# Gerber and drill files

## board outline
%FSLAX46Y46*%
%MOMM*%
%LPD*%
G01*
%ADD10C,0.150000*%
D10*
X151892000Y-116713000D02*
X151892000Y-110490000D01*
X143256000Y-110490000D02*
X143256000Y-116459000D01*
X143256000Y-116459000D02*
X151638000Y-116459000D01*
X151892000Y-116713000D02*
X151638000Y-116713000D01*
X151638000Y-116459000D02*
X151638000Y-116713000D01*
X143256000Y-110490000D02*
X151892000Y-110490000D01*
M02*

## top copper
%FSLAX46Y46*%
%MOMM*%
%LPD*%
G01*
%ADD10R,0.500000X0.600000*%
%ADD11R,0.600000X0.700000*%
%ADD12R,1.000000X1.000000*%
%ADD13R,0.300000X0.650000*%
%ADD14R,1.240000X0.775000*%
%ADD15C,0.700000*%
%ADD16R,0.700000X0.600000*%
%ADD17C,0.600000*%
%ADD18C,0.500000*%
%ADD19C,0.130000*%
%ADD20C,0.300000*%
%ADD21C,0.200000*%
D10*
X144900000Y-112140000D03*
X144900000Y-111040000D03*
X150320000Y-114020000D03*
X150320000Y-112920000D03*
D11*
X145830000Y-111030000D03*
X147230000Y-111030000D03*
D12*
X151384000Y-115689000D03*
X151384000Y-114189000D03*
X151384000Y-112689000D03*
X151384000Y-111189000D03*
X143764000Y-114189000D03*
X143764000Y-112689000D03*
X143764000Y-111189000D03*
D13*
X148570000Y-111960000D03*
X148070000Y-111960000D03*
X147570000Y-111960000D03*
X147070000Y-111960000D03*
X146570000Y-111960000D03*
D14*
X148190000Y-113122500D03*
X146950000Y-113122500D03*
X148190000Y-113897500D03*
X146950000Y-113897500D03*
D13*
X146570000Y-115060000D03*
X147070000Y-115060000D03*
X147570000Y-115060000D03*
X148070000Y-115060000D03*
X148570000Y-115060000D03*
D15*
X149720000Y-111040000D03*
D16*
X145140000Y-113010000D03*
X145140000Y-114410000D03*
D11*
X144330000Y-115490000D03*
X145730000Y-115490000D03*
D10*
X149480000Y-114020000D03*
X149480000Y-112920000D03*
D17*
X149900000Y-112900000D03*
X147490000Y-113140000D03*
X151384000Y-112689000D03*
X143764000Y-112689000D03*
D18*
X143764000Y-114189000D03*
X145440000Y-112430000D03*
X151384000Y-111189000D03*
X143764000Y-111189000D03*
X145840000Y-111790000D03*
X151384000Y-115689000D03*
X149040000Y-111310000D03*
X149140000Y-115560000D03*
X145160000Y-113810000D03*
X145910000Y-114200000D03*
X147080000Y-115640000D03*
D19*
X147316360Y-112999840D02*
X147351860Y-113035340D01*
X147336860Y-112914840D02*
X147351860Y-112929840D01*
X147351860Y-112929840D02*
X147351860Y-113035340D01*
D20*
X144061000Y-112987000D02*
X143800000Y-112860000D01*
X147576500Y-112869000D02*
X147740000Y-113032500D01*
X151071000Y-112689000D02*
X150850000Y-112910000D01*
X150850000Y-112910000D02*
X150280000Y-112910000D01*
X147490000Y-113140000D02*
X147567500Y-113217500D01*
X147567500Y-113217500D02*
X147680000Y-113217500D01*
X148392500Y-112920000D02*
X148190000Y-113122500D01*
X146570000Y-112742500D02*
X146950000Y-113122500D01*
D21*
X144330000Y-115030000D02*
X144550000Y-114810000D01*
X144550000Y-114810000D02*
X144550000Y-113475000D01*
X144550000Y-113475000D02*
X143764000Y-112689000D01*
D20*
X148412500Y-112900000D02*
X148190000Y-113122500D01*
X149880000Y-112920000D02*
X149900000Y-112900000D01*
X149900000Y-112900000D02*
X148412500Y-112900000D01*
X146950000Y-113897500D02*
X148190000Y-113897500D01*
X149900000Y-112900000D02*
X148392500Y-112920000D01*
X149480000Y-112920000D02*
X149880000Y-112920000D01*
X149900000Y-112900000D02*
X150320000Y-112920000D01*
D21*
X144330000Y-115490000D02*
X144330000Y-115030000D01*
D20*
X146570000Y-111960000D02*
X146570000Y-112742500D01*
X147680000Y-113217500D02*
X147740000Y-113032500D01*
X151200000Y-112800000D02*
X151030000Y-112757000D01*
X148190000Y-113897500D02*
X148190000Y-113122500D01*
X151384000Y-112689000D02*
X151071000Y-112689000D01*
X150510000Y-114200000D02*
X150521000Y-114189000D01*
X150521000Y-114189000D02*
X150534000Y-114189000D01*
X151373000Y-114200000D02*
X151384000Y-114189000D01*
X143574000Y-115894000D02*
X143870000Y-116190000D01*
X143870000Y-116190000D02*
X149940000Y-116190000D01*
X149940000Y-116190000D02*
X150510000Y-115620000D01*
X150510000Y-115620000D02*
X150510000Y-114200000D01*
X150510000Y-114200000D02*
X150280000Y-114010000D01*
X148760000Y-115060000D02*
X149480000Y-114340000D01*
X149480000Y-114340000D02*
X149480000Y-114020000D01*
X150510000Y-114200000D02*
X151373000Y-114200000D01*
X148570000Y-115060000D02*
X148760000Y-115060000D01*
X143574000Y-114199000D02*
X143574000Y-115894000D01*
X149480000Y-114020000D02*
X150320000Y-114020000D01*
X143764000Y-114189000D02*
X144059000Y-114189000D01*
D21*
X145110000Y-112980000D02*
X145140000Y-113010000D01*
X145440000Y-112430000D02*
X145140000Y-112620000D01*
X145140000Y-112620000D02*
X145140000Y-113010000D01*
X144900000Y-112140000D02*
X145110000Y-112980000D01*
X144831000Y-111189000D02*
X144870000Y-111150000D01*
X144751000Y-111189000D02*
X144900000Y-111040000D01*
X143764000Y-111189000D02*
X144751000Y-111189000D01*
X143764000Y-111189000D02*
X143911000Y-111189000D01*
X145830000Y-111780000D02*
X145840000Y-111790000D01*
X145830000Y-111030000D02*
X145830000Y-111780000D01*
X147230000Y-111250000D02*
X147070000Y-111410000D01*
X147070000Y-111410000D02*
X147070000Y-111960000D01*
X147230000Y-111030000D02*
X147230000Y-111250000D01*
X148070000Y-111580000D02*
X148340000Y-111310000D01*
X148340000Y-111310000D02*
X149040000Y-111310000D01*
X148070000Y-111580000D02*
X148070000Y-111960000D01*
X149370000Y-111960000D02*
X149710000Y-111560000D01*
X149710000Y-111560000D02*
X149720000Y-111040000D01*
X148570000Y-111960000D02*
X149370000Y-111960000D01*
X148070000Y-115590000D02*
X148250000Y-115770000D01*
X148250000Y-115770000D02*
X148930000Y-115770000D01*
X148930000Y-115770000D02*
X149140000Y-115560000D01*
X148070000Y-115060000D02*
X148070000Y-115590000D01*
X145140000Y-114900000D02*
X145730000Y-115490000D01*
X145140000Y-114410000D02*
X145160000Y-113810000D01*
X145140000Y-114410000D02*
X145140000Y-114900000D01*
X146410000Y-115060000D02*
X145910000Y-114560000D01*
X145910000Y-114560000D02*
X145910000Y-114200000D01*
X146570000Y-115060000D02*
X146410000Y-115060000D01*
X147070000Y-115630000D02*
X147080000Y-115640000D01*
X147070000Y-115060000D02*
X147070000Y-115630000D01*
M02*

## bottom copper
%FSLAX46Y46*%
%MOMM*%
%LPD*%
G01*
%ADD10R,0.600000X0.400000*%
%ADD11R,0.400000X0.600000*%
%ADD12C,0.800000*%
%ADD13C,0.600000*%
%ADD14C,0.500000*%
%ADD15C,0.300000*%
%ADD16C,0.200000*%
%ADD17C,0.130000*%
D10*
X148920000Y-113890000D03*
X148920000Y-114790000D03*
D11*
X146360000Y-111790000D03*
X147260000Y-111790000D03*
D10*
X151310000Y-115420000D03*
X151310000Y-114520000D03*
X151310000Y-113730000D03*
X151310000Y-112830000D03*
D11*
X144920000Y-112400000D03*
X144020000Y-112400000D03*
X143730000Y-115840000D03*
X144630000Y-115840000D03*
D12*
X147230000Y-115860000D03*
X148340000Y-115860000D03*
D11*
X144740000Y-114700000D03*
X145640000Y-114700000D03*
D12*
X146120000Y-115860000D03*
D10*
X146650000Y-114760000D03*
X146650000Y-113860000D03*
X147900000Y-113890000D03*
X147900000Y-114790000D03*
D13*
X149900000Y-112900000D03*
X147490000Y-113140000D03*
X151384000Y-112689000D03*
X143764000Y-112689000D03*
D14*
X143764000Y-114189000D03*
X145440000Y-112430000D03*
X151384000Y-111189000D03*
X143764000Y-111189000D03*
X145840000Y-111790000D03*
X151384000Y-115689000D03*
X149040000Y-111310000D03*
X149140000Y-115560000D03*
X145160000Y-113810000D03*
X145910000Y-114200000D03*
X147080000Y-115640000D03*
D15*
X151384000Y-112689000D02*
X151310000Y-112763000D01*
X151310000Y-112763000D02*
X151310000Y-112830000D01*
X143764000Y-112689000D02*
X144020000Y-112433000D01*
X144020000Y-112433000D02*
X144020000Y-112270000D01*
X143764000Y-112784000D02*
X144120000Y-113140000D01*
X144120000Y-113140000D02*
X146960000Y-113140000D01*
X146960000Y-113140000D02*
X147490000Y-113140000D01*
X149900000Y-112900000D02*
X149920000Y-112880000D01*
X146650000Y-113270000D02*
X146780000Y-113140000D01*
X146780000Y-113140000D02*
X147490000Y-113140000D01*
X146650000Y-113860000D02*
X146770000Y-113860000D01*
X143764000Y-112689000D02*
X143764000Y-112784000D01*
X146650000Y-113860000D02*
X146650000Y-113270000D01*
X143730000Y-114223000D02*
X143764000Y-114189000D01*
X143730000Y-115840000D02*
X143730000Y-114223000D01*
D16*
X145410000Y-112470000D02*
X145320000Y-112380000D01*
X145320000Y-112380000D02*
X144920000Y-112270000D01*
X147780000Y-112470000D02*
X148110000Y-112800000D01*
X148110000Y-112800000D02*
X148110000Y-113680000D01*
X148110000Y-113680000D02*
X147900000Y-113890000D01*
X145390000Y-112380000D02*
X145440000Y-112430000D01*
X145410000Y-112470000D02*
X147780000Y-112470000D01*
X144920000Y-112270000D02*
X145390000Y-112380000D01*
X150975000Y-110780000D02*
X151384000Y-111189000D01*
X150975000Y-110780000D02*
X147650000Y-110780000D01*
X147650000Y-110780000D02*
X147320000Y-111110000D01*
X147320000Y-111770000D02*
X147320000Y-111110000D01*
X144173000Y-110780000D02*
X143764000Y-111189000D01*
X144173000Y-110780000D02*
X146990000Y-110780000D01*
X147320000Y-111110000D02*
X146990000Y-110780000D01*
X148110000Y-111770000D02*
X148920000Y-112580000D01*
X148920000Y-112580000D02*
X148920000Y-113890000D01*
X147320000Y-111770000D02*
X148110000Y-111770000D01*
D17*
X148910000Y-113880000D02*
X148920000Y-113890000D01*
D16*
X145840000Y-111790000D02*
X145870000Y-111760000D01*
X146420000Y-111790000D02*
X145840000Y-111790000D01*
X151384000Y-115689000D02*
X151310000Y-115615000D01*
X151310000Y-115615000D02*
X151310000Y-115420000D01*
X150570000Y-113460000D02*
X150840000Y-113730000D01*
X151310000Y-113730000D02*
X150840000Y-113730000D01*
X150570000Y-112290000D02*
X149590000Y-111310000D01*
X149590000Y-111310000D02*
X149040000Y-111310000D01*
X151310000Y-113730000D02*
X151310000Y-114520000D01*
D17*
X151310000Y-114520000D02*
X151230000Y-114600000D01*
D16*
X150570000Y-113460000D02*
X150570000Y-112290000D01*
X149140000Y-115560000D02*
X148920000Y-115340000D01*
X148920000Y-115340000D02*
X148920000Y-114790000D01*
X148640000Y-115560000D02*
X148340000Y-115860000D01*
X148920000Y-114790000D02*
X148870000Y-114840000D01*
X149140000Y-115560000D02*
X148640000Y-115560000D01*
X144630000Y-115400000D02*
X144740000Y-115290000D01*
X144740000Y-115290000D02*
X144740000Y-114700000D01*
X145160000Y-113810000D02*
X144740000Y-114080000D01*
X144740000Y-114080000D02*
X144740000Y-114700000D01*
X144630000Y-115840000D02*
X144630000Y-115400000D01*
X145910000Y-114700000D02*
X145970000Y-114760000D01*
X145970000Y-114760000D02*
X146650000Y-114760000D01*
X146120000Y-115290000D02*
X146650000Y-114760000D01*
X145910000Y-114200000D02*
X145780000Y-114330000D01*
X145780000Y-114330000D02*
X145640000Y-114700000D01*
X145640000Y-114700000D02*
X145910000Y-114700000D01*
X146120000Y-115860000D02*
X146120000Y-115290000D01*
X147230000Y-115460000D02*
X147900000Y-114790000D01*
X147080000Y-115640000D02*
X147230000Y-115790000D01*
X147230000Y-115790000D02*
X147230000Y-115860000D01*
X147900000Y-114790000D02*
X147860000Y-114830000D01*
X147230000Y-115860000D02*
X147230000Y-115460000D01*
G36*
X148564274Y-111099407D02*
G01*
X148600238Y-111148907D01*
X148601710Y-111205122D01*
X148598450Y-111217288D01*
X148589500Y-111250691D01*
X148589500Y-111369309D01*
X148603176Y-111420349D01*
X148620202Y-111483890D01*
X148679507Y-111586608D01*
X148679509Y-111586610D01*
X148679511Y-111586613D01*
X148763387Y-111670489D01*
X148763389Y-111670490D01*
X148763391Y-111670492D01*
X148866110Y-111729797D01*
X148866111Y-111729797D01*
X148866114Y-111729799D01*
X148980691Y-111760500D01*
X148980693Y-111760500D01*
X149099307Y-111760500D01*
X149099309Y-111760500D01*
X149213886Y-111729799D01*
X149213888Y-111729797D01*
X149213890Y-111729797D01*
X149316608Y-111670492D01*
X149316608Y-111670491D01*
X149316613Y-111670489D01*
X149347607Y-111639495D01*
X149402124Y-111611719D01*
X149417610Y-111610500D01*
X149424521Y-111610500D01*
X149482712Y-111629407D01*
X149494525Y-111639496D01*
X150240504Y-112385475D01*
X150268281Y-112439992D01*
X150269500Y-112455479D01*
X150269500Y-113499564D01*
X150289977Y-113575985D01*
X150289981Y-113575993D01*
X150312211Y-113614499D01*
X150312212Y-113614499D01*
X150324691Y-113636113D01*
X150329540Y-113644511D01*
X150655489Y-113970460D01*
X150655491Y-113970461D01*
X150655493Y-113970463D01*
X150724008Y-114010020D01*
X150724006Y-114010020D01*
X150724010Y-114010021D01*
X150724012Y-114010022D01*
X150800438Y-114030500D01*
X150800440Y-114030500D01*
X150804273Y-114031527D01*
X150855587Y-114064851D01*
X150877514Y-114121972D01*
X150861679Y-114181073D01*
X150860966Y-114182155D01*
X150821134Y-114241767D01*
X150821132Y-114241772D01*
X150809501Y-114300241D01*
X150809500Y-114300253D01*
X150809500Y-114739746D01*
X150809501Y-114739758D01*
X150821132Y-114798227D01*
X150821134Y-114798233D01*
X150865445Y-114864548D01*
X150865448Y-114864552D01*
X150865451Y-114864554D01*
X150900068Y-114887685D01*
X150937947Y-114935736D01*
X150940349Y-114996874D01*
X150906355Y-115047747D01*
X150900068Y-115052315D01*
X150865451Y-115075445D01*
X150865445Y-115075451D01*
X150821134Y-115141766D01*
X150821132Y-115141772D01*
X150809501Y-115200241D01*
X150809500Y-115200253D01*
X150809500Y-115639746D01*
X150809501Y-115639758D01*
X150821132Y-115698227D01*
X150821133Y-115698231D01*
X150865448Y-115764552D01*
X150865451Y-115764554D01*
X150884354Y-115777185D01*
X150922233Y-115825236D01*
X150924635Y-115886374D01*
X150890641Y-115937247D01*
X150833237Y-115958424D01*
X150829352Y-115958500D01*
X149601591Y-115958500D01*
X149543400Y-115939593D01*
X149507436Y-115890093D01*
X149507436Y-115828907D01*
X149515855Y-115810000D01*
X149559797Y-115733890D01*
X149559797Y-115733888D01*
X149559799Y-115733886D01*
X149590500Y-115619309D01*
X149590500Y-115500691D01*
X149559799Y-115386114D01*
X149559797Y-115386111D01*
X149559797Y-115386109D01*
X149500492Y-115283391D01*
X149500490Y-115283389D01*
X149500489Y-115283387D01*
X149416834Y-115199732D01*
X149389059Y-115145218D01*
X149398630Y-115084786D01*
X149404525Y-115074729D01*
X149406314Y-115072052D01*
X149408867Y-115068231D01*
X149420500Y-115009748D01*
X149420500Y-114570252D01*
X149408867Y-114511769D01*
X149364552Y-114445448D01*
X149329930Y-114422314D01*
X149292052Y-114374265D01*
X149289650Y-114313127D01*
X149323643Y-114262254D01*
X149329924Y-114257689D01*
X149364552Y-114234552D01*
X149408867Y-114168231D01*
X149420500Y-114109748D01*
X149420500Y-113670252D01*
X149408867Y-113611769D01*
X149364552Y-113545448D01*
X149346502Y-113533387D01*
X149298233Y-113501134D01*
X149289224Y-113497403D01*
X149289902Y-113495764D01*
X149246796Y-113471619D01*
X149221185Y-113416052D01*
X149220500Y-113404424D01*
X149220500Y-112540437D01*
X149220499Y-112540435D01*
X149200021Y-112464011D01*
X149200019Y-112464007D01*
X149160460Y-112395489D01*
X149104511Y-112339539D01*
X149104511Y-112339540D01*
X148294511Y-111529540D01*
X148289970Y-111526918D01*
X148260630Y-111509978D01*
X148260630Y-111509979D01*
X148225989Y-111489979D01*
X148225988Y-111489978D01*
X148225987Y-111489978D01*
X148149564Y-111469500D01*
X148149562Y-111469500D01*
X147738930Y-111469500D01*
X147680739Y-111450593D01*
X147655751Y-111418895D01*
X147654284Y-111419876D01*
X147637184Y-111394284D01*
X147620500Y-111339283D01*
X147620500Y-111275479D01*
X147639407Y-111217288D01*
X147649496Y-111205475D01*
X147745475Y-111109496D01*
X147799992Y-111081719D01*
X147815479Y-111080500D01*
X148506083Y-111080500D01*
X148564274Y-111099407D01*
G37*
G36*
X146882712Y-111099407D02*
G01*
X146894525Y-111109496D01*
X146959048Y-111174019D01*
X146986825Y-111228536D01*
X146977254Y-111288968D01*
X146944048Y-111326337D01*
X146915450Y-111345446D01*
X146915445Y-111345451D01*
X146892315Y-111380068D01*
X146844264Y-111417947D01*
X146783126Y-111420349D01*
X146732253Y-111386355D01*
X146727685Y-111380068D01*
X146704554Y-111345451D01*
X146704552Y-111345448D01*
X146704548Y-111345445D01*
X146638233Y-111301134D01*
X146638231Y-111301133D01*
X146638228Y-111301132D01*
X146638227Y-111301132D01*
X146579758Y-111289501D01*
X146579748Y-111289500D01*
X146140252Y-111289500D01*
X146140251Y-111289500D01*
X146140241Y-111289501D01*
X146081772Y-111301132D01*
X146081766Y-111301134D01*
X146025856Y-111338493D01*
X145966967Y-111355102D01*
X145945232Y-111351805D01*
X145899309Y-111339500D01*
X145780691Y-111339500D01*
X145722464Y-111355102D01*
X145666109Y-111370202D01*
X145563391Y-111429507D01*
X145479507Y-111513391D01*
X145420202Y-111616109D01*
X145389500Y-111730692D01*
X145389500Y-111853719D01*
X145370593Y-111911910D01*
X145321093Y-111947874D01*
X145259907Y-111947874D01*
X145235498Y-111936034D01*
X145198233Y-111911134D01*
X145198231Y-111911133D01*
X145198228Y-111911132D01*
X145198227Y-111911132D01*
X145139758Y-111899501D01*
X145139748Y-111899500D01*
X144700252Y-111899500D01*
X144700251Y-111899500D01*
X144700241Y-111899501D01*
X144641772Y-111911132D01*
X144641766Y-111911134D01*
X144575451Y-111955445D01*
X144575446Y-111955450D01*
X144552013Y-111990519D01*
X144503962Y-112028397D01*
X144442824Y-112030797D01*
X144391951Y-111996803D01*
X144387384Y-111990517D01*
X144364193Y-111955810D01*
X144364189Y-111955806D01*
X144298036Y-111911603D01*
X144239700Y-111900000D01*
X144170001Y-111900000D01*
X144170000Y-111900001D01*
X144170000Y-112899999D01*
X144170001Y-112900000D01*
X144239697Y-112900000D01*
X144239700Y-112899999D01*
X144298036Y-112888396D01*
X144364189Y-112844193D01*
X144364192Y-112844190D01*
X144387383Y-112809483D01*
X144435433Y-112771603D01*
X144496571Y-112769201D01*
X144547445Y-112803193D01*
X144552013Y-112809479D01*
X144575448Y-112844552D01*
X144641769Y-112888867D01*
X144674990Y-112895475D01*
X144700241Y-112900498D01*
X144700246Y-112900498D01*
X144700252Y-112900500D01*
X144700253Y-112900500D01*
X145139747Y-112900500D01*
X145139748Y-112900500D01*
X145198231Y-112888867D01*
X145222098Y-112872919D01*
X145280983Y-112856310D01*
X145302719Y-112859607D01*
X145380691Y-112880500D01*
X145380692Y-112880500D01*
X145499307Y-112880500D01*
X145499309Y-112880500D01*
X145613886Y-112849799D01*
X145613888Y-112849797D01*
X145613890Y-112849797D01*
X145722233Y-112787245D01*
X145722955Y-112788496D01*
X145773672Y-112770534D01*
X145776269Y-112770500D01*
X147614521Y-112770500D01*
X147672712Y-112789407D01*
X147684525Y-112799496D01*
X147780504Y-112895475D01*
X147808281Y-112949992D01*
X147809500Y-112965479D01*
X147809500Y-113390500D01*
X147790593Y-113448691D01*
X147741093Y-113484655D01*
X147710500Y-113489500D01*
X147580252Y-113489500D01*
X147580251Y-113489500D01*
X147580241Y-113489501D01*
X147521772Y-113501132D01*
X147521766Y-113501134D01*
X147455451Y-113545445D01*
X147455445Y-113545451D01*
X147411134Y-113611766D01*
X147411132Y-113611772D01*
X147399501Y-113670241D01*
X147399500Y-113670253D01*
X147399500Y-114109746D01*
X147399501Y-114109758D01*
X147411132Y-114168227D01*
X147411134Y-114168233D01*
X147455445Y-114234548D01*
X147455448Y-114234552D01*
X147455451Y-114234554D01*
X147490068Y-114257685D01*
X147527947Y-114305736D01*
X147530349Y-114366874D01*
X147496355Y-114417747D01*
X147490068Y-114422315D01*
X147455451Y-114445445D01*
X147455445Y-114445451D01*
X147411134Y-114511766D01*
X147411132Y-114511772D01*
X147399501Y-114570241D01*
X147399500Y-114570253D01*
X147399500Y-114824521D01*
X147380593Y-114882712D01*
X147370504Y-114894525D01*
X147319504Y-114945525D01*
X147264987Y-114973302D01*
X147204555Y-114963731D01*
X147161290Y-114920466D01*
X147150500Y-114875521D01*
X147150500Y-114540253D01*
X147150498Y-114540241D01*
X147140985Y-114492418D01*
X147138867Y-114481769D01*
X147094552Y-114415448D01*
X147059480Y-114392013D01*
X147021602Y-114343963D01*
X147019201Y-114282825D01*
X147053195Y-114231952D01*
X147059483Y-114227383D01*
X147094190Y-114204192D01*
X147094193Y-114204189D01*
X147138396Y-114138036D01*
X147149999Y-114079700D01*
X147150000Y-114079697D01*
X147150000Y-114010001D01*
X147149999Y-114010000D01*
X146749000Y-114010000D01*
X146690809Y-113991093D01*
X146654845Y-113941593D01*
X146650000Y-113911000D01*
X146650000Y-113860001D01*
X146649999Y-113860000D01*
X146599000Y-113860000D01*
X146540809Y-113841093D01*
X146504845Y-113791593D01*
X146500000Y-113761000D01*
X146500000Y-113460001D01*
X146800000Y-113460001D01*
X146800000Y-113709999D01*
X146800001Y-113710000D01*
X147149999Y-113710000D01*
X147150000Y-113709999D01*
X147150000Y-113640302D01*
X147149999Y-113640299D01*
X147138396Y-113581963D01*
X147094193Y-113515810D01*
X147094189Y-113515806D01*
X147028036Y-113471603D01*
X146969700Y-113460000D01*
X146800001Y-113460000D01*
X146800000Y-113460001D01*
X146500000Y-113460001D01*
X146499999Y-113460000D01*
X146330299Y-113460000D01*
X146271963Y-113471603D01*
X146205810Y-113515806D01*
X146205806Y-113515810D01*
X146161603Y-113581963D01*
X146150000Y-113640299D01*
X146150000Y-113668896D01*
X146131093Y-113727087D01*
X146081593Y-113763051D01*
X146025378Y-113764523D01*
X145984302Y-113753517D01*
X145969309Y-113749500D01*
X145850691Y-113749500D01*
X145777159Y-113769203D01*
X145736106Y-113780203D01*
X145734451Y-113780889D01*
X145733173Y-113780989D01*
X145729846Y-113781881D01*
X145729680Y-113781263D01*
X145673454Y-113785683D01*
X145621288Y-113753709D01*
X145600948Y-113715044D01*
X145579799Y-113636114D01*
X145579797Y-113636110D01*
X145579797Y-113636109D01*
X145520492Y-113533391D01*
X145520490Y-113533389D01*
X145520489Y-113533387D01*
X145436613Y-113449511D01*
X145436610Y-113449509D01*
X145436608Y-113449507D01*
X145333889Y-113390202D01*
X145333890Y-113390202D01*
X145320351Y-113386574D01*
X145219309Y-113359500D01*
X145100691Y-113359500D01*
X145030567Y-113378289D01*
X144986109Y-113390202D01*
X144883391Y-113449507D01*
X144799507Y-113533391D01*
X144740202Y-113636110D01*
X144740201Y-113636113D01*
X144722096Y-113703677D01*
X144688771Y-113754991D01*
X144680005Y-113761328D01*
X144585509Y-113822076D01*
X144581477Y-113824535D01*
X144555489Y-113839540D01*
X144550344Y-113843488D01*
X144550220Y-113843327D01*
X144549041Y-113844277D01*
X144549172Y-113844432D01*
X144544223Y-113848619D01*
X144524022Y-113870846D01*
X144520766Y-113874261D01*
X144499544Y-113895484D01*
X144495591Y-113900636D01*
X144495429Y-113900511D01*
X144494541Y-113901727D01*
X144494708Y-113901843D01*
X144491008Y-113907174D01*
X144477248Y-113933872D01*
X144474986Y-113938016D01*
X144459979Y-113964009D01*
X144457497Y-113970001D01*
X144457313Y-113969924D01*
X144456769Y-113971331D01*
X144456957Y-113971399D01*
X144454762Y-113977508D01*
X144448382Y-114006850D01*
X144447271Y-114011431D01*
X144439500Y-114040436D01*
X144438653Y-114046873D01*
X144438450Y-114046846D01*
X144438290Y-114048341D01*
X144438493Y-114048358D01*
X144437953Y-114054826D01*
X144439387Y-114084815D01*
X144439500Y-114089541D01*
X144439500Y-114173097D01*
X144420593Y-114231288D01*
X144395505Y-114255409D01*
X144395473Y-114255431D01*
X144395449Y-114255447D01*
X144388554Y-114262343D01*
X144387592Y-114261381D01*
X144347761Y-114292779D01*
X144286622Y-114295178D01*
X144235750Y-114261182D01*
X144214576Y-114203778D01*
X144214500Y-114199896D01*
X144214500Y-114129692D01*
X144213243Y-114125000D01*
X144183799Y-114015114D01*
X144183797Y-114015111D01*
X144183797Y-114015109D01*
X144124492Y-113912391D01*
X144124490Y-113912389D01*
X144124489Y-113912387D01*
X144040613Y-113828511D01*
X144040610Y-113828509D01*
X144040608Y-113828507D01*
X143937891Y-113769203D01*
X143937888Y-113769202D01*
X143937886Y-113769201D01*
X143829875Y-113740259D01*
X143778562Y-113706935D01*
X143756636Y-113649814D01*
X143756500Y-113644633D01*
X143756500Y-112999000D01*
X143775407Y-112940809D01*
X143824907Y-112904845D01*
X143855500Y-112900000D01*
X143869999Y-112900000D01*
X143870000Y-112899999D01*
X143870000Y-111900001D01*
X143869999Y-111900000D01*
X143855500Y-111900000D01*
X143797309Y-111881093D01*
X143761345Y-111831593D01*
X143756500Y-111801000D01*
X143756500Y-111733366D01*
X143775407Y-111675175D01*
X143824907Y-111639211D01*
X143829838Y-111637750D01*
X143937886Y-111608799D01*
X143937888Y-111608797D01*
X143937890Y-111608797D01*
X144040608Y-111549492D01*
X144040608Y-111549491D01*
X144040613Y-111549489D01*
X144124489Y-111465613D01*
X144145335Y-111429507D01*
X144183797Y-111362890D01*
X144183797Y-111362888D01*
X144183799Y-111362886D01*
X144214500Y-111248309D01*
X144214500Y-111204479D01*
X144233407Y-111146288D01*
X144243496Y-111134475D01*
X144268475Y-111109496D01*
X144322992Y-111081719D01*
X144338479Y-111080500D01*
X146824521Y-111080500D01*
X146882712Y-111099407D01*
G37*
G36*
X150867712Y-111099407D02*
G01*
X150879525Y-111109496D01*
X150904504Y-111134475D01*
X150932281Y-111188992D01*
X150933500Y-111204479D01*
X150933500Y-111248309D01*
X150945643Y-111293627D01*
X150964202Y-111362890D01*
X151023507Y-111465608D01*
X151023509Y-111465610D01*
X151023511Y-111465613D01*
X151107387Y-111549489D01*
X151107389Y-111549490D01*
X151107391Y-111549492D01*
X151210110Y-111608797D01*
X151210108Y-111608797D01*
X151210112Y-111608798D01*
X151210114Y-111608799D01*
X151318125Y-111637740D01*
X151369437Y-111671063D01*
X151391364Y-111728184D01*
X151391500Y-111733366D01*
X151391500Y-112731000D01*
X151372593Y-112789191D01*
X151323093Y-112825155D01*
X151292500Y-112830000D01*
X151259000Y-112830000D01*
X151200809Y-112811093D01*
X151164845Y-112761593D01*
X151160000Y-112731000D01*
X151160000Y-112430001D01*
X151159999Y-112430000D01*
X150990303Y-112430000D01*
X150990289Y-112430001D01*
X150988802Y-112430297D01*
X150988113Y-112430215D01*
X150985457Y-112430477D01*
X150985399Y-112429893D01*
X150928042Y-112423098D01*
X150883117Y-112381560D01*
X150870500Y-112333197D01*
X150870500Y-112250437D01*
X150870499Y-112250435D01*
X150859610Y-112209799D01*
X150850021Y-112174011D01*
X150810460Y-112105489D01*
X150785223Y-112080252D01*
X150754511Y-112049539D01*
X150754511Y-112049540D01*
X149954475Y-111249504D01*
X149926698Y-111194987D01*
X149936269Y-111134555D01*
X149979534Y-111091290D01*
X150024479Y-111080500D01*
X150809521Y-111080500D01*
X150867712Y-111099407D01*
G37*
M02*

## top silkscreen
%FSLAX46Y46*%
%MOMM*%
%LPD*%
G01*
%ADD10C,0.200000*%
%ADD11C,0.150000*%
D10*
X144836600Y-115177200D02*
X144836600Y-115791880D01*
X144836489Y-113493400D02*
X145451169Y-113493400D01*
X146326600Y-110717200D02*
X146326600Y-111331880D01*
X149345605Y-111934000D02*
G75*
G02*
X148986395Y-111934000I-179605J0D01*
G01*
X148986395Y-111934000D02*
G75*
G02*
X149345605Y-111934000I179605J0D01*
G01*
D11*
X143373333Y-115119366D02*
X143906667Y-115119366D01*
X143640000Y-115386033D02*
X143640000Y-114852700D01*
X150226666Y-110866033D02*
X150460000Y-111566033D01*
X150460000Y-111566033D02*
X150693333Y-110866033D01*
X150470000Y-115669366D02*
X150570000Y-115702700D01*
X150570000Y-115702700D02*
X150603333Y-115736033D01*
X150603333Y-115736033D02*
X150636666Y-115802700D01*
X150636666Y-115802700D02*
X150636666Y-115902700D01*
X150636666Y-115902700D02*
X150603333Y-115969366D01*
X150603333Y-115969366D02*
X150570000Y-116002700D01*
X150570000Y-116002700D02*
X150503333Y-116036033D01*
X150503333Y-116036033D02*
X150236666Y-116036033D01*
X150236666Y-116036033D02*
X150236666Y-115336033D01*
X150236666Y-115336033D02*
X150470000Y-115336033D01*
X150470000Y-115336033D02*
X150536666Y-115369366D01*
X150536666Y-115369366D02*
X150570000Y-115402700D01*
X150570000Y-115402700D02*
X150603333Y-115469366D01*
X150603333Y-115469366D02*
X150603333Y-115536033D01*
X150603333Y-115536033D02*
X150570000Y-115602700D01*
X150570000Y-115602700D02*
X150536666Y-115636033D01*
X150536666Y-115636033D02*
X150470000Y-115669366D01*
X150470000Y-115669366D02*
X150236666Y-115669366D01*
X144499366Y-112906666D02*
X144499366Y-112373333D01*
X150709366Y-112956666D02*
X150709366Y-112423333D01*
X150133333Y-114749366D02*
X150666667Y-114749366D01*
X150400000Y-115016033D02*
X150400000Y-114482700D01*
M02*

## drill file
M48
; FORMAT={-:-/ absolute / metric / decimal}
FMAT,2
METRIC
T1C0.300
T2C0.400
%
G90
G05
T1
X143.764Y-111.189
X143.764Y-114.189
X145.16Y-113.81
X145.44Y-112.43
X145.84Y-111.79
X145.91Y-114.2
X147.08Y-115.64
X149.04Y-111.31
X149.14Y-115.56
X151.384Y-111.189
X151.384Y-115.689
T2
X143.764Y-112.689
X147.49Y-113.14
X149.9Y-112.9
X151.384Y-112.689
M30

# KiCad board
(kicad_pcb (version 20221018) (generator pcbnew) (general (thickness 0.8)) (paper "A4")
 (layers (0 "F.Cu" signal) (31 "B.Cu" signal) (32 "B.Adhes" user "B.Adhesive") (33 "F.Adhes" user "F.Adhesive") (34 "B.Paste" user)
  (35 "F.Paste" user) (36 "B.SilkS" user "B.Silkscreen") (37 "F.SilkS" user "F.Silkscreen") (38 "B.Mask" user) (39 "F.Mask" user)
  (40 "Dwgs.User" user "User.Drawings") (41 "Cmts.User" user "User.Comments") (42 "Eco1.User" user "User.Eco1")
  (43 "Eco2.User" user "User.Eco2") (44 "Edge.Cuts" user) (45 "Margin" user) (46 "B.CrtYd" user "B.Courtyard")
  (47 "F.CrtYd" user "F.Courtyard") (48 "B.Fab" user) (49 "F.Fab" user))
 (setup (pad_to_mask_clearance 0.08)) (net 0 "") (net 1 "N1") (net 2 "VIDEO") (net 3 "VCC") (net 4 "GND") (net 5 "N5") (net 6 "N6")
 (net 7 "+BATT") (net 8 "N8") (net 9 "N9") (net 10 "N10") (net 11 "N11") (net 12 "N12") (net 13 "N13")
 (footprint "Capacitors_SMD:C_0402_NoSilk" (layer "F.Cu") (at 144.9 111.59 90)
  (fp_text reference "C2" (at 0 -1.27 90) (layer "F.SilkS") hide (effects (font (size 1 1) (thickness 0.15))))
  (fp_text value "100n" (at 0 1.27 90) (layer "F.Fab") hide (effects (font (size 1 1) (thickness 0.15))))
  (pad "1" smd rect (at -0.55 0 90) (size 0.6 0.5) (layers "F.Cu" "F.Paste" "F.Mask") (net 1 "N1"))
  (pad "2" smd rect (at 0.55 0 90) (size 0.6 0.5) (layers "F.Cu" "F.Paste" "F.Mask") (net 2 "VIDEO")))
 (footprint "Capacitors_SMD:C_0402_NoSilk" (layer "F.Cu") (at 150.32 113.47 90)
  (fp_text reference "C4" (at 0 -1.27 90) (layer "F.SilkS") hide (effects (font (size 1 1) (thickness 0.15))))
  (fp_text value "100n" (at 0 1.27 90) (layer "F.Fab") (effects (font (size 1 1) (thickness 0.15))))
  (pad "1" smd rect (at -0.55 0 90) (size 0.6 0.5) (layers "F.Cu" "F.Paste" "F.Mask") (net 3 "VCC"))
  (pad "2" smd rect (at 0.55 0 90) (size 0.6 0.5) (layers "F.Cu" "F.Paste" "F.Mask") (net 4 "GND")))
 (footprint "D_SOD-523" (layer "F.Cu") (at 146.53 111.03)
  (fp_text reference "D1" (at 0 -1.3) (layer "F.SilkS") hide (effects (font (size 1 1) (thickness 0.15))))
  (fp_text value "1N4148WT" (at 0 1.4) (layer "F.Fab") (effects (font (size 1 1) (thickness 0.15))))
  (pad "1" smd rect (at -0.7 0 180) (size 0.6 0.7) (layers "F.Cu" "F.Paste" "F.Mask") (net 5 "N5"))
  (pad "2" smd rect (at 0.7 0 180) (size 0.6 0.7) (layers "F.Cu" "F.Paste" "F.Mask") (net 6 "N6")))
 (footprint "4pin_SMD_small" (layer "F.Cu") (at 151.384 115.189 90)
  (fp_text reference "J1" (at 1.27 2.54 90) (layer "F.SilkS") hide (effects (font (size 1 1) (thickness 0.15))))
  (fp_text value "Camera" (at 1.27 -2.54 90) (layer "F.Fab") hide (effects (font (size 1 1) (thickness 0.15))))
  (pad "1" smd rect (at -0.5 0 90) (size 1 1) (layers "F.Cu" "F.Paste" "F.Mask") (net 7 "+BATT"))
  (pad "2" smd rect (at 1 0 90) (size 1 1) (layers "F.Cu" "F.Paste" "F.Mask") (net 3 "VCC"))
  (pad "3" smd rect (at 2.5 0 90) (size 1 1) (layers "F.Cu" "F.Paste" "F.Mask") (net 4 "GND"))
  (pad "4" smd rect (at 4 0 90) (size 1 1) (layers "F.Cu" "F.Paste" "F.Mask") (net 2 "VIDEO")))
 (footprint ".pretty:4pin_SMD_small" (layer "F.Cu") (at 143.764 115.189 90)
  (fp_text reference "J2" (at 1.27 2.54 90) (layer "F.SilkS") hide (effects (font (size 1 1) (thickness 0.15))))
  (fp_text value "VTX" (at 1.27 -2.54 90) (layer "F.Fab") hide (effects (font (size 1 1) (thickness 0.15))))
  (pad "2" smd rect (at 1 0 90) (size 1 1) (layers "F.Cu" "F.Paste" "F.Mask") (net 3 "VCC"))
  (pad "3" smd rect (at 2.5 0 90) (size 1 1) (layers "F.Cu" "F.Paste" "F.Mask") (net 4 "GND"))
  (pad "4" smd rect (at 4 0 90) (size 1 1) (layers "F.Cu" "F.Paste" "F.Mask") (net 2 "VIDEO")))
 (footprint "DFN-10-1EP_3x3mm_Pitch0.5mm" (layer "F.Cu") (at 147.57 113.51 -90)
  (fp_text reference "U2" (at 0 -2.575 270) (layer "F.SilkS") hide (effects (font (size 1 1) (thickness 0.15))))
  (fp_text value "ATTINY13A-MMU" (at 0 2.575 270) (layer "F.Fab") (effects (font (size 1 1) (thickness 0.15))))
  (pad "1" smd rect (at -1.55 -1 270) (size 0.65 0.3) (layers "F.Cu" "F.Paste" "F.Mask") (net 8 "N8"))
  (pad "2" smd rect (at -1.55 -0.5 270) (size 0.65 0.3) (layers "F.Cu" "F.Paste" "F.Mask") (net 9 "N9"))
  (pad "3" smd rect (at -1.55 0 270) (size 0.65 0.3) (layers "F.Cu" "F.Paste" "F.Mask"))
  (pad "4" smd rect (at -1.55 0.5 270) (size 0.65 0.3) (layers "F.Cu" "F.Paste" "F.Mask") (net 6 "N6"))
  (pad "5" smd rect (at -1.55 1 270) (size 0.65 0.3) (layers "F.Cu" "F.Paste" "F.Mask") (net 4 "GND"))
  (pad "5" smd rect (at -0.3875 -0.62 270) (size 0.775 1.24) (layers "F.Cu" "F.Paste" "F.Mask") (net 4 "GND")
   (solder_paste_margin_ratio -0.2))
  (pad "5" smd rect (at -0.3875 0.62 270) (size 0.775 1.24) (layers "F.Cu" "F.Paste" "F.Mask") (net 4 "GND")
   (solder_paste_margin_ratio -0.2))
  (pad "5" smd rect (at 0.3875 -0.62 270) (size 0.775 1.24) (layers "F.Cu" "F.Paste" "F.Mask") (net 4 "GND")
   (solder_paste_margin_ratio -0.2))
  (pad "5" smd rect (at 0.3875 0.62 270) (size 0.775 1.24) (layers "F.Cu" "F.Paste" "F.Mask") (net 4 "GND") (solder_paste_margin_ratio -0.2))
  (pad "6" smd rect (at 1.55 1 270) (size 0.65 0.3) (layers "F.Cu" "F.Paste" "F.Mask") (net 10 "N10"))
  (pad "7" smd rect (at 1.55 0.5 270) (size 0.65 0.3) (layers "F.Cu" "F.Paste" "F.Mask") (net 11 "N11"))
  (pad "8" smd rect (at 1.55 0 270) (size 0.65 0.3) (layers "F.Cu" "F.Paste" "F.Mask"))
  (pad "9" smd rect (at 1.55 -0.5 270) (size 0.65 0.3) (layers "F.Cu" "F.Paste" "F.Mask") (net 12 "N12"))
  (pad "10" smd rect (at 1.55 -1 270) (size 0.65 0.3) (layers "F.Cu" "F.Paste" "F.Mask") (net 3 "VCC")))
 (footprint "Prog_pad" (layer "F.Cu") (at 149.72 111.04)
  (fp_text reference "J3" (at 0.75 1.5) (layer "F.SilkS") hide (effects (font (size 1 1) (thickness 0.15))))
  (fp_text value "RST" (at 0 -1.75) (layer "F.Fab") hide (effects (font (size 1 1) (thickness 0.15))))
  (pad "1" smd circle (at 0 0) (size 0.7 0.7) (layers "F.Cu" "F.Paste" "F.Mask") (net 8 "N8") (solder_mask_margin 0.02)))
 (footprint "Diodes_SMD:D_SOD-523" (layer "F.Cu") (at 145.14 113.71 -90)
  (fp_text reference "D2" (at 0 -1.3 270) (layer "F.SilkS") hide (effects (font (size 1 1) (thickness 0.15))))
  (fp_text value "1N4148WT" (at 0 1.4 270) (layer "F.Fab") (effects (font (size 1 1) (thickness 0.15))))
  (pad "1" smd rect (at -0.7 0 90) (size 0.6 0.7) (layers "F.Cu" "F.Paste" "F.Mask") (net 1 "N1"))
  (pad "2" smd rect (at 0.7 0 90) (size 0.6 0.7) (layers "F.Cu" "F.Paste" "F.Mask") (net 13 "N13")))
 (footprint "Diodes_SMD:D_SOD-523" (layer "F.Cu") (at 145.03 115.49)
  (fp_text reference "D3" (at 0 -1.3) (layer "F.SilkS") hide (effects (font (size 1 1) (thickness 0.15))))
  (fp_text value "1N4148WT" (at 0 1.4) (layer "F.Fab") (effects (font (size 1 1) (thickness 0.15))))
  (pad "1" smd rect (at -0.7 0 180) (size 0.6 0.7) (layers "F.Cu" "F.Paste" "F.Mask") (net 4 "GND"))
  (pad "2" smd rect (at 0.7 0 180) (size 0.6 0.7) (layers "F.Cu" "F.Paste" "F.Mask") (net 13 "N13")))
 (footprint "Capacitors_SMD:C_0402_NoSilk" (layer "F.Cu") (at 149.48 113.47 90)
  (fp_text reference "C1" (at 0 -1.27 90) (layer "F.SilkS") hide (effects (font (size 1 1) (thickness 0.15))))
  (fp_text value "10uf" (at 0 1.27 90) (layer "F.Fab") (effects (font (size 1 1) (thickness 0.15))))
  (pad "1" smd rect (at -0.55 0 90) (size 0.6 0.5) (layers "F.Cu" "F.Paste" "F.Mask") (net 3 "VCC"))
  (pad "2" smd rect (at 0.55 0 90) (size 0.6 0.5) (layers "F.Cu" "F.Paste" "F.Mask") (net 4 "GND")))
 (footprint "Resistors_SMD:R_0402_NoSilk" (layer "B.Cu") (at 148.92 114.34 -90)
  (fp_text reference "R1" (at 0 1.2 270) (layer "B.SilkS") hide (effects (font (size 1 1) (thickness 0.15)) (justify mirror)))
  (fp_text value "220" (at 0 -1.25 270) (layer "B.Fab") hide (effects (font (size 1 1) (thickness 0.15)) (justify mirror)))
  (pad "1" smd rect (at -0.45 0 270) (size 0.4 0.6) (layers "B.Cu" "B.Paste" "B.Mask") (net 2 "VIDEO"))
  (pad "2" smd rect (at 0.45 0 270) (size 0.4 0.6) (layers "B.Cu" "B.Paste" "B.Mask") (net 12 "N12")))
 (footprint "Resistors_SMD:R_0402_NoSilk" (layer "B.Cu") (at 146.81 111.79)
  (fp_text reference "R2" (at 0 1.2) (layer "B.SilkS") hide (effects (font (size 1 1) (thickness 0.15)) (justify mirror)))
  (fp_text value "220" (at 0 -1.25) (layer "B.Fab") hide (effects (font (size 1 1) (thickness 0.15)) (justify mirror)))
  (pad "1" smd rect (at -0.45 0) (size 0.4 0.6) (layers "B.Cu" "B.Paste" "B.Mask") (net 5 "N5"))
  (pad "2" smd rect (at 0.45 0) (size 0.4 0.6) (layers "B.Cu" "B.Paste" "B.Mask") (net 2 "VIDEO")))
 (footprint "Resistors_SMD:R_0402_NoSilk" (layer "B.Cu") (at 151.31 114.97 90)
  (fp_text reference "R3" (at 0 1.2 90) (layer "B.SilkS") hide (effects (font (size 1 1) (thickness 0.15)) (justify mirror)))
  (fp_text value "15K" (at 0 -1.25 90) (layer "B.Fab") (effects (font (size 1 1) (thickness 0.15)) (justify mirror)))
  (pad "1" smd rect (at -0.45 0 90) (size 0.4 0.6) (layers "B.Cu" "B.Paste" "B.Mask") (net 7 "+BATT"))
  (pad "2" smd rect (at 0.45 0 90) (size 0.4 0.6) (layers "B.Cu" "B.Paste" "B.Mask") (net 9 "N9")))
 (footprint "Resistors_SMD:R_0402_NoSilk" (layer "B.Cu") (at 151.31 113.28 90)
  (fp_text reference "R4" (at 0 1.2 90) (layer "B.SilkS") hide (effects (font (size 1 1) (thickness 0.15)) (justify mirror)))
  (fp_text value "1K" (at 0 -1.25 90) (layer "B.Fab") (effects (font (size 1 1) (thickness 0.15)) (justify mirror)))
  (pad "1" smd rect (at -0.45 0 90) (size 0.4 0.6) (layers "B.Cu" "B.Paste" "B.Mask") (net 9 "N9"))
  (pad "2" smd rect (at 0.45 0 90) (size 0.4 0.6) (layers "B.Cu" "B.Paste" "B.Mask") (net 4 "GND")))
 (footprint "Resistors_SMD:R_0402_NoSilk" (layer "B.Cu") (at 144.47 112.4 180)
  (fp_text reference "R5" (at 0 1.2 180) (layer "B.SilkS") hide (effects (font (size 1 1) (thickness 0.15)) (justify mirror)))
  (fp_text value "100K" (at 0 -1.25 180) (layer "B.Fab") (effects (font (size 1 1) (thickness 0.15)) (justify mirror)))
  (pad "1" smd rect (at -0.45 0 180) (size 0.4 0.6) (layers "B.Cu" "B.Paste" "B.Mask") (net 1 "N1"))
  (pad "2" smd rect (at 0.45 0 180) (size 0.4 0.6) (layers "B.Cu" "B.Paste" "B.Mask") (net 4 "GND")))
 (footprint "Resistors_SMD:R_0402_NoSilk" (layer "B.Cu") (at 144.18 115.84)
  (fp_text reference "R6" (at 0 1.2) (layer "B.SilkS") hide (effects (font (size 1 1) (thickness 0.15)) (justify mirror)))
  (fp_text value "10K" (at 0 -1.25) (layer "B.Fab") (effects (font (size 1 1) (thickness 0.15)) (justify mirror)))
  (pad "1" smd rect (at -0.45 0) (size 0.4 0.6) (layers "B.Cu" "B.Paste" "B.Mask") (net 3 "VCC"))
  (pad "2" smd rect (at 0.45 0) (size 0.4 0.6) (layers "B.Cu" "B.Paste" "B.Mask") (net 13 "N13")))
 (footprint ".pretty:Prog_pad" (layer "B.Cu") (at 147.23 115.86)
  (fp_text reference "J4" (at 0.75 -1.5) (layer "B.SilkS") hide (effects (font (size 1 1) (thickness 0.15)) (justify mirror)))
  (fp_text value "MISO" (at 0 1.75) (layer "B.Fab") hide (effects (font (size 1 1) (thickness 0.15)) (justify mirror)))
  (pad "1" smd circle (at 0 0) (size 0.8 0.8) (layers "B.Cu" "B.Paste" "B.Mask") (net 11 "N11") (solder_mask_margin 0.02)))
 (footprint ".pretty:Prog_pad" (layer "B.Cu") (at 148.34 115.86)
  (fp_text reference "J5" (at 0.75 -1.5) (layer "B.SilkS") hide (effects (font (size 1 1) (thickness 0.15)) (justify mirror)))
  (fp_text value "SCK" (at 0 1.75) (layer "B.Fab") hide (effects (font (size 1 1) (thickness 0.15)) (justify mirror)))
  (pad "1" smd circle (at 0 0) (size 0.8 0.8) (layers "B.Cu" "B.Paste" "B.Mask") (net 12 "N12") (solder_mask_margin 0.02)))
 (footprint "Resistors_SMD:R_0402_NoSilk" (layer "B.Cu") (at 145.19 114.7)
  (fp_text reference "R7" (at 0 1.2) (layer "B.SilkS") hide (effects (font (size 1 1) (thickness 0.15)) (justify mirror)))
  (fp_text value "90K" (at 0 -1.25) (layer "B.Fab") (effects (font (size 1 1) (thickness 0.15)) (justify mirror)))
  (pad "1" smd rect (at -0.45 0) (size 0.4 0.6) (layers "B.Cu" "B.Paste" "B.Mask") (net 13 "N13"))
  (pad "2" smd rect (at 0.45 0) (size 0.4 0.6) (layers "B.Cu" "B.Paste" "B.Mask") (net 10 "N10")))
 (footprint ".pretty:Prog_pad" (layer "B.Cu") (at 146.12 115.86)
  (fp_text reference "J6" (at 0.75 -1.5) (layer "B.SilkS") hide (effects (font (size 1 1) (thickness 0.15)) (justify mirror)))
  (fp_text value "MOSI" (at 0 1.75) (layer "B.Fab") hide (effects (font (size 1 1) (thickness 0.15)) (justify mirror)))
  (pad "1" smd circle (at 0 0) (size 0.8 0.8) (layers "B.Cu" "B.Paste" "B.Mask") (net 10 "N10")))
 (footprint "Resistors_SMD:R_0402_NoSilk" (layer "B.Cu") (at 146.65 114.31 90)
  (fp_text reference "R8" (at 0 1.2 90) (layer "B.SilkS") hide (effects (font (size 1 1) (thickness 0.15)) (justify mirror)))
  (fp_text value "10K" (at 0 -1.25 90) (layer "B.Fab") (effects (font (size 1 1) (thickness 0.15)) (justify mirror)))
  (pad "1" smd rect (at -0.45 0 90) (size 0.4 0.6) (layers "B.Cu" "B.Paste" "B.Mask") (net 10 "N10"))
  (pad "2" smd rect (at 0.45 0 90) (size 0.4 0.6) (layers "B.Cu" "B.Paste" "B.Mask") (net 4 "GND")))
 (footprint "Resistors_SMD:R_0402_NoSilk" (layer "B.Cu") (at 147.9 114.34 -90)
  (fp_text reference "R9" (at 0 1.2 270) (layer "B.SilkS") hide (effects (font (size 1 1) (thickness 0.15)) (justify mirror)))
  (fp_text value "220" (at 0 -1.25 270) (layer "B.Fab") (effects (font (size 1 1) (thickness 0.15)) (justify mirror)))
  (pad "1" smd rect (at -0.45 0 270) (size 0.4 0.6) (layers "B.Cu" "B.Paste" "B.Mask") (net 1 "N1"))
  (pad "2" smd rect (at 0.45 0 270) (size 0.4 0.6) (layers "B.Cu" "B.Paste" "B.Mask") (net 11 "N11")))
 (gr_line (start 144.8366 115.1772) (end 144.8366 115.79188) (stroke (width 0.2) (type solid)) (layer "F.SilkS"))
 (gr_line (start 144.836489 113.4934) (end 145.451169 113.4934) (stroke (width 0.2) (type solid)) (layer "F.SilkS"))
 (gr_line (start 146.3266 110.7172) (end 146.3266 111.33188) (stroke (width 0.2) (type solid)) (layer "F.SilkS"))
 (gr_circle (center 149.166 111.934) (end 149.039 111.807) (stroke (width 0.2) (type solid)) (fill none) (layer "F.SilkS"))
 (gr_line (start 151.892 116.713) (end 151.892 110.49) (stroke (width 0.15) (type solid)) (layer "Edge.Cuts"))
 (gr_line (start 143.256 110.49) (end 143.256 116.459) (stroke (width 0.15) (type solid)) (layer "Edge.Cuts"))
 (gr_line (start 143.256 116.459) (end 151.638 116.459) (stroke (width 0.15) (type solid)) (layer "Edge.Cuts"))
 (gr_line (start 151.892 116.713) (end 151.638 116.713) (stroke (width 0.15) (type solid)) (layer "Edge.Cuts"))
 (gr_line (start 151.638 116.459) (end 151.638 116.713) (stroke (width 0.15) (type solid)) (layer "Edge.Cuts"))
 (gr_line (start 143.256 110.49) (end 151.892 110.49) (stroke (width 0.15) (type solid)) (layer "Edge.Cuts"))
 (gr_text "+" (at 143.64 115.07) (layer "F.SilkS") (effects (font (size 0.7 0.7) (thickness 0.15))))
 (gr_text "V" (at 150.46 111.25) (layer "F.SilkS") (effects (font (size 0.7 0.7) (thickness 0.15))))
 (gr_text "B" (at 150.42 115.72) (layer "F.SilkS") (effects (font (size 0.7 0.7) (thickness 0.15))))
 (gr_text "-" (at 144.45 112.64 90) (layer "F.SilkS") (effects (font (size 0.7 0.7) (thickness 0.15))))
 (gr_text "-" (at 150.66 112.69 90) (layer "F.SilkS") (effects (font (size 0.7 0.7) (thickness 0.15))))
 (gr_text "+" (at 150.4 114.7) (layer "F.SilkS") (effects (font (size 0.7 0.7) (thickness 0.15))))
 (segment (start 147.31636 112.99984) (end 147.35186 113.03534) (width 0.13) (layer "F.Cu") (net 4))
 (segment (start 147.33686 112.91484) (end 147.35186 112.92984) (width 0.13) (layer "F.Cu") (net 4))
 (segment (start 147.35186 112.92984) (end 147.35186 113.03534) (width 0.13) (layer "F.Cu") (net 4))
 (segment (start 144.061 112.987) (end 143.8 112.86) (width 0.3) (layer "F.Cu") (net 4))
 (segment (start 147.5765 112.869) (end 147.74 113.0325) (width 0.3) (layer "F.Cu") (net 4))
 (segment (start 151.071 112.689) (end 150.85 112.91) (width 0.3) (layer "F.Cu") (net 4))
 (segment (start 150.85 112.91) (end 150.28 112.91) (width 0.3) (layer "F.Cu") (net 4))
 (segment (start 147.49 113.14) (end 147.5675 113.2175) (width 0.3) (layer "F.Cu") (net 4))
 (segment (start 147.5675 113.2175) (end 147.68 113.2175) (width 0.3) (layer "F.Cu") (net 4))
 (segment (start 148.3925 112.92) (end 148.19 113.1225) (width 0.3) (layer "F.Cu") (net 4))
 (segment (start 146.57 112.7425) (end 146.95 113.1225) (width 0.3) (layer "F.Cu") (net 4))
 (segment (start 144.33 115.03) (end 144.55 114.81) (width 0.2) (layer "F.Cu") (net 4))
 (segment (start 144.55 114.81) (end 144.55 113.475) (width 0.2) (layer "F.Cu") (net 4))
 (segment (start 144.55 113.475) (end 143.764 112.689) (width 0.2) (layer "F.Cu") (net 4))
 (segment (start 148.4125 112.9) (end 148.19 113.1225) (width 0.3) (layer "F.Cu") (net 4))
 (segment (start 149.88 112.92) (end 149.9 112.9) (width 0.3) (layer "F.Cu") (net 4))
 (segment (start 149.9 112.9) (end 148.4125 112.9) (width 0.3) (layer "F.Cu") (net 4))
 (segment (start 146.95 113.8975) (end 148.19 113.8975) (width 0.3) (layer "F.Cu") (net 4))
 (segment (start 149.9 112.9) (end 148.3925 112.92) (width 0.3) (layer "F.Cu") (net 4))
 (segment (start 149.48 112.92) (end 149.88 112.92) (width 0.3) (layer "F.Cu") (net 4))
 (segment (start 149.9 112.9) (end 150.32 112.92) (width 0.3) (layer "F.Cu") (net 4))
 (segment (start 144.33 115.49) (end 144.33 115.03) (width 0.2) (layer "F.Cu") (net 4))
 (segment (start 146.57 111.96) (end 146.57 112.7425) (width 0.3) (layer "F.Cu") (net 4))
 (segment (start 147.68 113.2175) (end 147.74 113.0325) (width 0.3) (layer "F.Cu") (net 4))
 (segment (start 151.2 112.8) (end 151.03 112.757) (width 0.3) (layer "F.Cu") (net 4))
 (segment (start 148.19 113.8975) (end 148.19 113.1225) (width 0.3) (layer "F.Cu") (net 4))
 (segment (start 151.384 112.689) (end 151.071 112.689) (width 0.3) (layer "F.Cu") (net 4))
 (via (at 149.9 112.9) (size 0.6) (drill 0.4) (layers "F.Cu" "B.Cu") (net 4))
 (via (at 147.49 113.14) (size 0.6) (drill 0.4) (layers "F.Cu" "B.Cu") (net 4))
 (via (at 151.384 112.689) (size 0.6) (drill 0.4) (layers "F.Cu" "B.Cu") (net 4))
 (via (at 143.764 112.689) (size 0.6) (drill 0.4) (layers "F.Cu" "B.Cu") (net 4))
 (segment (start 151.384 112.689) (end 151.31 112.763) (width 0.3) (layer "B.Cu") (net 4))
 (segment (start 151.31 112.763) (end 151.31 112.83) (width 0.3) (layer "B.Cu") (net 4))
 (segment (start 143.764 112.689) (end 144.02 112.433) (width 0.3) (layer "B.Cu") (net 4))
 (segment (start 144.02 112.433) (end 144.02 112.27) (width 0.3) (layer "B.Cu") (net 4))
 (segment (start 143.764 112.784) (end 144.12 113.14) (width 0.3) (layer "B.Cu") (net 4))
 (segment (start 144.12 113.14) (end 146.96 113.14) (width 0.3) (layer "B.Cu") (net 4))
 (segment (start 146.96 113.14) (end 147.49 113.14) (width 0.3) (layer "B.Cu") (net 4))
 (segment (start 149.9 112.9) (end 149.92 112.88) (width 0.3) (layer "B.Cu") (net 4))
 (segment (start 146.65 113.27) (end 146.78 113.14) (width 0.3) (layer "B.Cu") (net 4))
 (segment (start 146.78 113.14) (end 147.49 113.14) (width 0.3) (layer "B.Cu") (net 4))
 (segment (start 146.65 113.86) (end 146.77 113.86) (width 0.3) (layer "B.Cu") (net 4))
 (segment (start 143.764 112.689) (end 143.764 112.784) (width 0.3) (layer "B.Cu") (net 4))
 (segment (start 146.65 113.86) (end 146.65 113.27) (width 0.3) (layer "B.Cu") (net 4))
 (segment (start 150.51 114.2) (end 150.521 114.189) (width 0.3) (layer "F.Cu") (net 3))
 (segment (start 150.521 114.189) (end 150.534 114.189) (width 0.3) (layer "F.Cu") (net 3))
 (segment (start 151.373 114.2) (end 151.384 114.189) (width 0.3) (layer "F.Cu") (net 3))
 (segment (start 143.574 115.894) (end 143.87 116.19) (width 0.3) (layer "F.Cu") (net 3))
 (segment (start 143.87 116.19) (end 149.94 116.19) (width 0.3) (layer "F.Cu") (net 3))
 (segment (start 149.94 116.19) (end 150.51 115.62) (width 0.3) (layer "F.Cu") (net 3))
 (segment (start 150.51 115.62) (end 150.51 114.2) (width 0.3) (layer "F.Cu") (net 3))
 (segment (start 150.51 114.2) (end 150.28 114.01) (width 0.3) (layer "F.Cu") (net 3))
 (segment (start 148.76 115.06) (end 149.48 114.34) (width 0.3) (layer "F.Cu") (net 3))
 (segment (start 149.48 114.34) (end 149.48 114.02) (width 0.3) (layer "F.Cu") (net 3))
 (segment (start 150.51 114.2) (end 151.373 114.2) (width 0.3) (layer "F.Cu") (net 3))
 (segment (start 148.57 115.06) (end 148.76 115.06) (width 0.3) (layer "F.Cu") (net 3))
 (segment (start 143.574 114.199) (end 143.574 115.894) (width 0.3) (layer "F.Cu") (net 3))
 (segment (start 149.48 114.02) (end 150.32 114.02) (width 0.3) (layer "F.Cu") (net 3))
 (segment (start 143.764 114.189) (end 144.059 114.189) (width 0.3) (layer "F.Cu") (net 3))
 (via (at 143.764 114.189) (size 0.5) (drill 0.3) (layers "F.Cu" "B.Cu") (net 3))
 (segment (start 143.73 114.223) (end 143.764 114.189) (width 0.3) (layer "B.Cu") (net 3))
 (segment (start 143.73 115.84) (end 143.73 114.223) (width 0.3) (layer "B.Cu") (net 3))
 (segment (start 145.11 112.98) (end 145.14 113.01) (width 0.2) (layer "F.Cu") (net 1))
 (segment (start 145.44 112.43) (end 145.14 112.62) (width 0.2) (layer "F.Cu") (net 1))
 (segment (start 145.14 112.62) (end 145.14 113.01) (width 0.2) (layer "F.Cu") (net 1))
 (segment (start 144.9 112.14) (end 145.11 112.98) (width 0.2) (layer "F.Cu") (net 1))
 (via (at 145.44 112.43) (size 0.5) (drill 0.3) (layers "F.Cu" "B.Cu") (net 1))
 (segment (start 145.41 112.47) (end 145.32 112.38) (width 0.2) (layer "B.Cu") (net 1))
 (segment (start 145.32 112.38) (end 144.92 112.27) (width 0.2) (layer "B.Cu") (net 1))
 (segment (start 147.78 112.47) (end 148.11 112.8) (width 0.2) (layer "B.Cu") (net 1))
 (segment (start 148.11 112.8) (end 148.11 113.68) (width 0.2) (layer "B.Cu") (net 1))
 (segment (start 148.11 113.68) (end 147.9 113.89) (width 0.2) (layer "B.Cu") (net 1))
 (segment (start 145.39 112.38) (end 145.44 112.43) (width 0.2) (layer "B.Cu") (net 1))
 (segment (start 145.41 112.47) (end 147.78 112.47) (width 0.2) (layer "B.Cu") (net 1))
 (segment (start 144.92 112.27) (end 145.39 112.38) (width 0.2) (layer "B.Cu") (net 1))
 (segment (start 144.831 111.189) (end 144.87 111.15) (width 0.2) (layer "F.Cu") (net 2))
 (segment (start 144.751 111.189) (end 144.9 111.04) (width 0.2) (layer "F.Cu") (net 2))
 (segment (start 143.764 111.189) (end 144.751 111.189) (width 0.2) (layer "F.Cu") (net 2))
 (segment (start 143.764 111.189) (end 143.911 111.189) (width 0.2) (layer "F.Cu") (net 2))
 (via (at 151.384 111.189) (size 0.5) (drill 0.3) (layers "F.Cu" "B.Cu") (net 2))
 (via (at 143.764 111.189) (size 0.5) (drill 0.3) (layers "F.Cu" "B.Cu") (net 2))
 (segment (start 150.975 110.78) (end 151.384 111.189) (width 0.2) (layer "B.Cu") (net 2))
 (segment (start 150.975 110.78) (end 147.65 110.78) (width 0.2) (layer "B.Cu") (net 2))
 (segment (start 147.65 110.78) (end 147.32 111.11) (width 0.2) (layer "B.Cu") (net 2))
 (segment (start 147.32 111.77) (end 147.32 111.11) (width 0.2) (layer "B.Cu") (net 2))
 (segment (start 144.173 110.78) (end 143.764 111.189) (width 0.2) (layer "B.Cu") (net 2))
 (segment (start 144.173 110.78) (end 146.99 110.78) (width 0.2) (layer "B.Cu") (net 2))
 (segment (start 147.32 111.11) (end 146.99 110.78) (width 0.2) (layer "B.Cu") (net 2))
 (segment (start 148.11 111.77) (end 148.92 112.58) (width 0.2) (layer "B.Cu") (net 2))
 (segment (start 148.92 112.58) (end 148.92 113.89) (width 0.2) (layer "B.Cu") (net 2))
 (segment (start 147.32 111.77) (end 148.11 111.77) (width 0.2) (layer "B.Cu") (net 2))
 (segment (start 148.91 113.88) (end 148.92 113.89) (width 0.13) (layer "B.Cu") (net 2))
 (segment (start 145.83 111.78) (end 145.84 111.79) (width 0.2) (layer "F.Cu") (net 5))
 (segment (start 145.83 111.03) (end 145.83 111.78) (width 0.2) (layer "F.Cu") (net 5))
 (via (at 145.84 111.79) (size 0.5) (drill 0.3) (layers "F.Cu" "B.Cu") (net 5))
 (segment (start 145.84 111.79) (end 145.87 111.76) (width 0.2) (layer "B.Cu") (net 5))
 (segment (start 146.42 111.79) (end 145.84 111.79) (width 0.2) (layer "B.Cu") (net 5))
 (segment (start 147.23 111.25) (end 147.07 111.41) (width 0.2) (layer "F.Cu") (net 6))
 (segment (start 147.07 111.41) (end 147.07 111.96) (width 0.2) (layer "F.Cu") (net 6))
 (segment (start 147.23 111.03) (end 147.23 111.25) (width 0.2) (layer "F.Cu") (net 6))
 (via (at 151.384 115.689) (size 0.5) (drill 0.3) (layers "F.Cu" "B.Cu") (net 7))
 (segment (start 151.384 115.689) (end 151.31 115.615) (width 0.2) (layer "B.Cu") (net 7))
 (segment (start 151.31 115.615) (end 151.31 115.42) (width 0.2) (layer "B.Cu") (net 7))
 (segment (start 148.07 111.58) (end 148.34 111.31) (width 0.2) (layer "F.Cu") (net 9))
 (segment (start 148.34 111.31) (end 149.04 111.31) (width 0.2) (layer "F.Cu") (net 9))
 (segment (start 148.07 111.58) (end 148.07 111.96) (width 0.2) (layer "F.Cu") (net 9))
 (via (at 149.04 111.31) (size 0.5) (drill 0.3) (layers "F.Cu" "B.Cu") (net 9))
 (segment (start 150.57 113.46) (end 150.84 113.73) (width 0.2) (layer "B.Cu") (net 9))
 (segment (start 151.31 113.73) (end 150.84 113.73) (width 0.2) (layer "B.Cu") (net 9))
 (segment (start 150.57 112.29) (end 149.59 111.31) (width 0.2) (layer "B.Cu") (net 9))
 (segment (start 149.59 111.31) (end 149.04 111.31) (width 0.2) (layer "B.Cu") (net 9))
 (segment (start 151.31 113.73) (end 151.31 114.52) (width 0.2) (layer "B.Cu") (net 9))
 (segment (start 151.31 114.52) (end 151.23 114.6) (width 0.13) (layer "B.Cu") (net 9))
 (segment (start 150.57 113.46) (end 150.57 112.29) (width 0.2) (layer "B.Cu") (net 9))
 (segment (start 149.37 111.96) (end 149.71 111.56) (width 0.2) (layer "F.Cu") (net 8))
 (segment (start 149.71 111.56) (end 149.72 111.04) (width 0.2) (layer "F.Cu") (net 8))
 (segment (start 148.57 111.96) (end 149.37 111.96) (width 0.2) (layer "F.Cu") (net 8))
 (segment (start 148.07 115.59) (end 148.25 115.77) (width 0.2) (layer "F.Cu") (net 12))
 (segment (start 148.25 115.77) (end 148.93 115.77) (width 0.2) (layer "F.Cu") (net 12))
 (segment (start 148.93 115.77) (end 149.14 115.56) (width 0.2) (layer "F.Cu") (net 12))
 (segment (start 148.07 115.06) (end 148.07 115.59) (width 0.2) (layer "F.Cu") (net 12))
 (via (at 149.14 115.56) (size 0.5) (drill 0.3) (layers "F.Cu" "B.Cu") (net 12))
 (segment (start 149.14 115.56) (end 148.92 115.34) (width 0.2) (layer "B.Cu") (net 12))
 (segment (start 148.92 115.34) (end 148.92 114.79) (width 0.2) (layer "B.Cu") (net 12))
 (segment (start 148.64 115.56) (end 148.34 115.86) (width 0.2) (layer "B.Cu") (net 12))
 (segment (start 148.92 114.79) (end 148.87 114.84) (width 0.2) (layer "B.Cu") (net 12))
 (segment (start 149.14 115.56) (end 148.64 115.56) (width 0.2) (layer "B.Cu") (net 12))
 (segment (start 145.14 114.9) (end 145.73 115.49) (width 0.2) (layer "F.Cu") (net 13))
 (segment (start 145.14 114.41) (end 145.16 113.81) (width 0.2) (layer "F.Cu") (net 13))
 (segment (start 145.14 114.41) (end 145.14 114.9) (width 0.2) (layer "F.Cu") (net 13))
 (via (at 145.16 113.81) (size 0.5) (drill 0.3) (layers "F.Cu" "B.Cu") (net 13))
 (segment (start 144.63 115.4) (end 144.74 115.29) (width 0.2) (layer "B.Cu") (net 13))
 (segment (start 144.74 115.29) (end 144.74 114.7) (width 0.2) (layer "B.Cu") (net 13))
 (segment (start 145.16 113.81) (end 144.74 114.08) (width 0.2) (layer "B.Cu") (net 13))
 (segment (start 144.74 114.08) (end 144.74 114.7) (width 0.2) (layer "B.Cu") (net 13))
 (segment (start 144.63 115.84) (end 144.63 115.4) (width 0.2) (layer "B.Cu") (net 13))
 (segment (start 146.41 115.06) (end 145.91 114.56) (width 0.2) (layer "F.Cu") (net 10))
 (segment (start 145.91 114.56) (end 145.91 114.2) (width 0.2) (layer "F.Cu") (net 10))
 (segment (start 146.57 115.06) (end 146.41 115.06) (width 0.2) (layer "F.Cu") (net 10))
 (via (at 145.91 114.2) (size 0.5) (drill 0.3) (layers "F.Cu" "B.Cu") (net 10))
 (segment (start 145.91 114.7) (end 145.97 114.76) (width 0.2) (layer "B.Cu") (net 10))
 (segment (start 145.97 114.76) (end 146.65 114.76) (width 0.2) (layer "B.Cu") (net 10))
 (segment (start 146.12 115.29) (end 146.65 114.76) (width 0.2) (layer "B.Cu") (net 10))
 (segment (start 145.91 114.2) (end 145.78 114.33) (width 0.2) (layer "B.Cu") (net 10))
 (segment (start 145.78 114.33) (end 145.64 114.7) (width 0.2) (layer "B.Cu") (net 10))
 (segment (start 145.64 114.7) (end 145.91 114.7) (width 0.2) (layer "B.Cu") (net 10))
 (segment (start 146.12 115.86) (end 146.12 115.29) (width 0.2) (layer "B.Cu") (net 10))
 (segment (start 147.07 115.63) (end 147.08 115.64) (width 0.2) (layer "F.Cu") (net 11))
 (segment (start 147.07 115.06) (end 147.07 115.63) (width 0.2) (layer "F.Cu") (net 11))
 (via (at 147.08 115.64) (size 0.5) (drill 0.3) (layers "F.Cu" "B.Cu") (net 11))
 (segment (start 147.23 115.46) (end 147.9 114.79) (width 0.2) (layer "B.Cu") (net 11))
 (segment (start 147.08 115.64) (end 147.23 115.79) (width 0.2) (layer "B.Cu") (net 11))
 (segment (start 147.23 115.79) (end 147.23 115.86) (width 0.2) (layer "B.Cu") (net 11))
 (segment (start 147.9 114.79) (end 147.86 114.83) (width 0.2) (layer "B.Cu") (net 11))
 (segment (start 147.23 115.86) (end 147.23 115.46) (width 0.2) (layer "B.Cu") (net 11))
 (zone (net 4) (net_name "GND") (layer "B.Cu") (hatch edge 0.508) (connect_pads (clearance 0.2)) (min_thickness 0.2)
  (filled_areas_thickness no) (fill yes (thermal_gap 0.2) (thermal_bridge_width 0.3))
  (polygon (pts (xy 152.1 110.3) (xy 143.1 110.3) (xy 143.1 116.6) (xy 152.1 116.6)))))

